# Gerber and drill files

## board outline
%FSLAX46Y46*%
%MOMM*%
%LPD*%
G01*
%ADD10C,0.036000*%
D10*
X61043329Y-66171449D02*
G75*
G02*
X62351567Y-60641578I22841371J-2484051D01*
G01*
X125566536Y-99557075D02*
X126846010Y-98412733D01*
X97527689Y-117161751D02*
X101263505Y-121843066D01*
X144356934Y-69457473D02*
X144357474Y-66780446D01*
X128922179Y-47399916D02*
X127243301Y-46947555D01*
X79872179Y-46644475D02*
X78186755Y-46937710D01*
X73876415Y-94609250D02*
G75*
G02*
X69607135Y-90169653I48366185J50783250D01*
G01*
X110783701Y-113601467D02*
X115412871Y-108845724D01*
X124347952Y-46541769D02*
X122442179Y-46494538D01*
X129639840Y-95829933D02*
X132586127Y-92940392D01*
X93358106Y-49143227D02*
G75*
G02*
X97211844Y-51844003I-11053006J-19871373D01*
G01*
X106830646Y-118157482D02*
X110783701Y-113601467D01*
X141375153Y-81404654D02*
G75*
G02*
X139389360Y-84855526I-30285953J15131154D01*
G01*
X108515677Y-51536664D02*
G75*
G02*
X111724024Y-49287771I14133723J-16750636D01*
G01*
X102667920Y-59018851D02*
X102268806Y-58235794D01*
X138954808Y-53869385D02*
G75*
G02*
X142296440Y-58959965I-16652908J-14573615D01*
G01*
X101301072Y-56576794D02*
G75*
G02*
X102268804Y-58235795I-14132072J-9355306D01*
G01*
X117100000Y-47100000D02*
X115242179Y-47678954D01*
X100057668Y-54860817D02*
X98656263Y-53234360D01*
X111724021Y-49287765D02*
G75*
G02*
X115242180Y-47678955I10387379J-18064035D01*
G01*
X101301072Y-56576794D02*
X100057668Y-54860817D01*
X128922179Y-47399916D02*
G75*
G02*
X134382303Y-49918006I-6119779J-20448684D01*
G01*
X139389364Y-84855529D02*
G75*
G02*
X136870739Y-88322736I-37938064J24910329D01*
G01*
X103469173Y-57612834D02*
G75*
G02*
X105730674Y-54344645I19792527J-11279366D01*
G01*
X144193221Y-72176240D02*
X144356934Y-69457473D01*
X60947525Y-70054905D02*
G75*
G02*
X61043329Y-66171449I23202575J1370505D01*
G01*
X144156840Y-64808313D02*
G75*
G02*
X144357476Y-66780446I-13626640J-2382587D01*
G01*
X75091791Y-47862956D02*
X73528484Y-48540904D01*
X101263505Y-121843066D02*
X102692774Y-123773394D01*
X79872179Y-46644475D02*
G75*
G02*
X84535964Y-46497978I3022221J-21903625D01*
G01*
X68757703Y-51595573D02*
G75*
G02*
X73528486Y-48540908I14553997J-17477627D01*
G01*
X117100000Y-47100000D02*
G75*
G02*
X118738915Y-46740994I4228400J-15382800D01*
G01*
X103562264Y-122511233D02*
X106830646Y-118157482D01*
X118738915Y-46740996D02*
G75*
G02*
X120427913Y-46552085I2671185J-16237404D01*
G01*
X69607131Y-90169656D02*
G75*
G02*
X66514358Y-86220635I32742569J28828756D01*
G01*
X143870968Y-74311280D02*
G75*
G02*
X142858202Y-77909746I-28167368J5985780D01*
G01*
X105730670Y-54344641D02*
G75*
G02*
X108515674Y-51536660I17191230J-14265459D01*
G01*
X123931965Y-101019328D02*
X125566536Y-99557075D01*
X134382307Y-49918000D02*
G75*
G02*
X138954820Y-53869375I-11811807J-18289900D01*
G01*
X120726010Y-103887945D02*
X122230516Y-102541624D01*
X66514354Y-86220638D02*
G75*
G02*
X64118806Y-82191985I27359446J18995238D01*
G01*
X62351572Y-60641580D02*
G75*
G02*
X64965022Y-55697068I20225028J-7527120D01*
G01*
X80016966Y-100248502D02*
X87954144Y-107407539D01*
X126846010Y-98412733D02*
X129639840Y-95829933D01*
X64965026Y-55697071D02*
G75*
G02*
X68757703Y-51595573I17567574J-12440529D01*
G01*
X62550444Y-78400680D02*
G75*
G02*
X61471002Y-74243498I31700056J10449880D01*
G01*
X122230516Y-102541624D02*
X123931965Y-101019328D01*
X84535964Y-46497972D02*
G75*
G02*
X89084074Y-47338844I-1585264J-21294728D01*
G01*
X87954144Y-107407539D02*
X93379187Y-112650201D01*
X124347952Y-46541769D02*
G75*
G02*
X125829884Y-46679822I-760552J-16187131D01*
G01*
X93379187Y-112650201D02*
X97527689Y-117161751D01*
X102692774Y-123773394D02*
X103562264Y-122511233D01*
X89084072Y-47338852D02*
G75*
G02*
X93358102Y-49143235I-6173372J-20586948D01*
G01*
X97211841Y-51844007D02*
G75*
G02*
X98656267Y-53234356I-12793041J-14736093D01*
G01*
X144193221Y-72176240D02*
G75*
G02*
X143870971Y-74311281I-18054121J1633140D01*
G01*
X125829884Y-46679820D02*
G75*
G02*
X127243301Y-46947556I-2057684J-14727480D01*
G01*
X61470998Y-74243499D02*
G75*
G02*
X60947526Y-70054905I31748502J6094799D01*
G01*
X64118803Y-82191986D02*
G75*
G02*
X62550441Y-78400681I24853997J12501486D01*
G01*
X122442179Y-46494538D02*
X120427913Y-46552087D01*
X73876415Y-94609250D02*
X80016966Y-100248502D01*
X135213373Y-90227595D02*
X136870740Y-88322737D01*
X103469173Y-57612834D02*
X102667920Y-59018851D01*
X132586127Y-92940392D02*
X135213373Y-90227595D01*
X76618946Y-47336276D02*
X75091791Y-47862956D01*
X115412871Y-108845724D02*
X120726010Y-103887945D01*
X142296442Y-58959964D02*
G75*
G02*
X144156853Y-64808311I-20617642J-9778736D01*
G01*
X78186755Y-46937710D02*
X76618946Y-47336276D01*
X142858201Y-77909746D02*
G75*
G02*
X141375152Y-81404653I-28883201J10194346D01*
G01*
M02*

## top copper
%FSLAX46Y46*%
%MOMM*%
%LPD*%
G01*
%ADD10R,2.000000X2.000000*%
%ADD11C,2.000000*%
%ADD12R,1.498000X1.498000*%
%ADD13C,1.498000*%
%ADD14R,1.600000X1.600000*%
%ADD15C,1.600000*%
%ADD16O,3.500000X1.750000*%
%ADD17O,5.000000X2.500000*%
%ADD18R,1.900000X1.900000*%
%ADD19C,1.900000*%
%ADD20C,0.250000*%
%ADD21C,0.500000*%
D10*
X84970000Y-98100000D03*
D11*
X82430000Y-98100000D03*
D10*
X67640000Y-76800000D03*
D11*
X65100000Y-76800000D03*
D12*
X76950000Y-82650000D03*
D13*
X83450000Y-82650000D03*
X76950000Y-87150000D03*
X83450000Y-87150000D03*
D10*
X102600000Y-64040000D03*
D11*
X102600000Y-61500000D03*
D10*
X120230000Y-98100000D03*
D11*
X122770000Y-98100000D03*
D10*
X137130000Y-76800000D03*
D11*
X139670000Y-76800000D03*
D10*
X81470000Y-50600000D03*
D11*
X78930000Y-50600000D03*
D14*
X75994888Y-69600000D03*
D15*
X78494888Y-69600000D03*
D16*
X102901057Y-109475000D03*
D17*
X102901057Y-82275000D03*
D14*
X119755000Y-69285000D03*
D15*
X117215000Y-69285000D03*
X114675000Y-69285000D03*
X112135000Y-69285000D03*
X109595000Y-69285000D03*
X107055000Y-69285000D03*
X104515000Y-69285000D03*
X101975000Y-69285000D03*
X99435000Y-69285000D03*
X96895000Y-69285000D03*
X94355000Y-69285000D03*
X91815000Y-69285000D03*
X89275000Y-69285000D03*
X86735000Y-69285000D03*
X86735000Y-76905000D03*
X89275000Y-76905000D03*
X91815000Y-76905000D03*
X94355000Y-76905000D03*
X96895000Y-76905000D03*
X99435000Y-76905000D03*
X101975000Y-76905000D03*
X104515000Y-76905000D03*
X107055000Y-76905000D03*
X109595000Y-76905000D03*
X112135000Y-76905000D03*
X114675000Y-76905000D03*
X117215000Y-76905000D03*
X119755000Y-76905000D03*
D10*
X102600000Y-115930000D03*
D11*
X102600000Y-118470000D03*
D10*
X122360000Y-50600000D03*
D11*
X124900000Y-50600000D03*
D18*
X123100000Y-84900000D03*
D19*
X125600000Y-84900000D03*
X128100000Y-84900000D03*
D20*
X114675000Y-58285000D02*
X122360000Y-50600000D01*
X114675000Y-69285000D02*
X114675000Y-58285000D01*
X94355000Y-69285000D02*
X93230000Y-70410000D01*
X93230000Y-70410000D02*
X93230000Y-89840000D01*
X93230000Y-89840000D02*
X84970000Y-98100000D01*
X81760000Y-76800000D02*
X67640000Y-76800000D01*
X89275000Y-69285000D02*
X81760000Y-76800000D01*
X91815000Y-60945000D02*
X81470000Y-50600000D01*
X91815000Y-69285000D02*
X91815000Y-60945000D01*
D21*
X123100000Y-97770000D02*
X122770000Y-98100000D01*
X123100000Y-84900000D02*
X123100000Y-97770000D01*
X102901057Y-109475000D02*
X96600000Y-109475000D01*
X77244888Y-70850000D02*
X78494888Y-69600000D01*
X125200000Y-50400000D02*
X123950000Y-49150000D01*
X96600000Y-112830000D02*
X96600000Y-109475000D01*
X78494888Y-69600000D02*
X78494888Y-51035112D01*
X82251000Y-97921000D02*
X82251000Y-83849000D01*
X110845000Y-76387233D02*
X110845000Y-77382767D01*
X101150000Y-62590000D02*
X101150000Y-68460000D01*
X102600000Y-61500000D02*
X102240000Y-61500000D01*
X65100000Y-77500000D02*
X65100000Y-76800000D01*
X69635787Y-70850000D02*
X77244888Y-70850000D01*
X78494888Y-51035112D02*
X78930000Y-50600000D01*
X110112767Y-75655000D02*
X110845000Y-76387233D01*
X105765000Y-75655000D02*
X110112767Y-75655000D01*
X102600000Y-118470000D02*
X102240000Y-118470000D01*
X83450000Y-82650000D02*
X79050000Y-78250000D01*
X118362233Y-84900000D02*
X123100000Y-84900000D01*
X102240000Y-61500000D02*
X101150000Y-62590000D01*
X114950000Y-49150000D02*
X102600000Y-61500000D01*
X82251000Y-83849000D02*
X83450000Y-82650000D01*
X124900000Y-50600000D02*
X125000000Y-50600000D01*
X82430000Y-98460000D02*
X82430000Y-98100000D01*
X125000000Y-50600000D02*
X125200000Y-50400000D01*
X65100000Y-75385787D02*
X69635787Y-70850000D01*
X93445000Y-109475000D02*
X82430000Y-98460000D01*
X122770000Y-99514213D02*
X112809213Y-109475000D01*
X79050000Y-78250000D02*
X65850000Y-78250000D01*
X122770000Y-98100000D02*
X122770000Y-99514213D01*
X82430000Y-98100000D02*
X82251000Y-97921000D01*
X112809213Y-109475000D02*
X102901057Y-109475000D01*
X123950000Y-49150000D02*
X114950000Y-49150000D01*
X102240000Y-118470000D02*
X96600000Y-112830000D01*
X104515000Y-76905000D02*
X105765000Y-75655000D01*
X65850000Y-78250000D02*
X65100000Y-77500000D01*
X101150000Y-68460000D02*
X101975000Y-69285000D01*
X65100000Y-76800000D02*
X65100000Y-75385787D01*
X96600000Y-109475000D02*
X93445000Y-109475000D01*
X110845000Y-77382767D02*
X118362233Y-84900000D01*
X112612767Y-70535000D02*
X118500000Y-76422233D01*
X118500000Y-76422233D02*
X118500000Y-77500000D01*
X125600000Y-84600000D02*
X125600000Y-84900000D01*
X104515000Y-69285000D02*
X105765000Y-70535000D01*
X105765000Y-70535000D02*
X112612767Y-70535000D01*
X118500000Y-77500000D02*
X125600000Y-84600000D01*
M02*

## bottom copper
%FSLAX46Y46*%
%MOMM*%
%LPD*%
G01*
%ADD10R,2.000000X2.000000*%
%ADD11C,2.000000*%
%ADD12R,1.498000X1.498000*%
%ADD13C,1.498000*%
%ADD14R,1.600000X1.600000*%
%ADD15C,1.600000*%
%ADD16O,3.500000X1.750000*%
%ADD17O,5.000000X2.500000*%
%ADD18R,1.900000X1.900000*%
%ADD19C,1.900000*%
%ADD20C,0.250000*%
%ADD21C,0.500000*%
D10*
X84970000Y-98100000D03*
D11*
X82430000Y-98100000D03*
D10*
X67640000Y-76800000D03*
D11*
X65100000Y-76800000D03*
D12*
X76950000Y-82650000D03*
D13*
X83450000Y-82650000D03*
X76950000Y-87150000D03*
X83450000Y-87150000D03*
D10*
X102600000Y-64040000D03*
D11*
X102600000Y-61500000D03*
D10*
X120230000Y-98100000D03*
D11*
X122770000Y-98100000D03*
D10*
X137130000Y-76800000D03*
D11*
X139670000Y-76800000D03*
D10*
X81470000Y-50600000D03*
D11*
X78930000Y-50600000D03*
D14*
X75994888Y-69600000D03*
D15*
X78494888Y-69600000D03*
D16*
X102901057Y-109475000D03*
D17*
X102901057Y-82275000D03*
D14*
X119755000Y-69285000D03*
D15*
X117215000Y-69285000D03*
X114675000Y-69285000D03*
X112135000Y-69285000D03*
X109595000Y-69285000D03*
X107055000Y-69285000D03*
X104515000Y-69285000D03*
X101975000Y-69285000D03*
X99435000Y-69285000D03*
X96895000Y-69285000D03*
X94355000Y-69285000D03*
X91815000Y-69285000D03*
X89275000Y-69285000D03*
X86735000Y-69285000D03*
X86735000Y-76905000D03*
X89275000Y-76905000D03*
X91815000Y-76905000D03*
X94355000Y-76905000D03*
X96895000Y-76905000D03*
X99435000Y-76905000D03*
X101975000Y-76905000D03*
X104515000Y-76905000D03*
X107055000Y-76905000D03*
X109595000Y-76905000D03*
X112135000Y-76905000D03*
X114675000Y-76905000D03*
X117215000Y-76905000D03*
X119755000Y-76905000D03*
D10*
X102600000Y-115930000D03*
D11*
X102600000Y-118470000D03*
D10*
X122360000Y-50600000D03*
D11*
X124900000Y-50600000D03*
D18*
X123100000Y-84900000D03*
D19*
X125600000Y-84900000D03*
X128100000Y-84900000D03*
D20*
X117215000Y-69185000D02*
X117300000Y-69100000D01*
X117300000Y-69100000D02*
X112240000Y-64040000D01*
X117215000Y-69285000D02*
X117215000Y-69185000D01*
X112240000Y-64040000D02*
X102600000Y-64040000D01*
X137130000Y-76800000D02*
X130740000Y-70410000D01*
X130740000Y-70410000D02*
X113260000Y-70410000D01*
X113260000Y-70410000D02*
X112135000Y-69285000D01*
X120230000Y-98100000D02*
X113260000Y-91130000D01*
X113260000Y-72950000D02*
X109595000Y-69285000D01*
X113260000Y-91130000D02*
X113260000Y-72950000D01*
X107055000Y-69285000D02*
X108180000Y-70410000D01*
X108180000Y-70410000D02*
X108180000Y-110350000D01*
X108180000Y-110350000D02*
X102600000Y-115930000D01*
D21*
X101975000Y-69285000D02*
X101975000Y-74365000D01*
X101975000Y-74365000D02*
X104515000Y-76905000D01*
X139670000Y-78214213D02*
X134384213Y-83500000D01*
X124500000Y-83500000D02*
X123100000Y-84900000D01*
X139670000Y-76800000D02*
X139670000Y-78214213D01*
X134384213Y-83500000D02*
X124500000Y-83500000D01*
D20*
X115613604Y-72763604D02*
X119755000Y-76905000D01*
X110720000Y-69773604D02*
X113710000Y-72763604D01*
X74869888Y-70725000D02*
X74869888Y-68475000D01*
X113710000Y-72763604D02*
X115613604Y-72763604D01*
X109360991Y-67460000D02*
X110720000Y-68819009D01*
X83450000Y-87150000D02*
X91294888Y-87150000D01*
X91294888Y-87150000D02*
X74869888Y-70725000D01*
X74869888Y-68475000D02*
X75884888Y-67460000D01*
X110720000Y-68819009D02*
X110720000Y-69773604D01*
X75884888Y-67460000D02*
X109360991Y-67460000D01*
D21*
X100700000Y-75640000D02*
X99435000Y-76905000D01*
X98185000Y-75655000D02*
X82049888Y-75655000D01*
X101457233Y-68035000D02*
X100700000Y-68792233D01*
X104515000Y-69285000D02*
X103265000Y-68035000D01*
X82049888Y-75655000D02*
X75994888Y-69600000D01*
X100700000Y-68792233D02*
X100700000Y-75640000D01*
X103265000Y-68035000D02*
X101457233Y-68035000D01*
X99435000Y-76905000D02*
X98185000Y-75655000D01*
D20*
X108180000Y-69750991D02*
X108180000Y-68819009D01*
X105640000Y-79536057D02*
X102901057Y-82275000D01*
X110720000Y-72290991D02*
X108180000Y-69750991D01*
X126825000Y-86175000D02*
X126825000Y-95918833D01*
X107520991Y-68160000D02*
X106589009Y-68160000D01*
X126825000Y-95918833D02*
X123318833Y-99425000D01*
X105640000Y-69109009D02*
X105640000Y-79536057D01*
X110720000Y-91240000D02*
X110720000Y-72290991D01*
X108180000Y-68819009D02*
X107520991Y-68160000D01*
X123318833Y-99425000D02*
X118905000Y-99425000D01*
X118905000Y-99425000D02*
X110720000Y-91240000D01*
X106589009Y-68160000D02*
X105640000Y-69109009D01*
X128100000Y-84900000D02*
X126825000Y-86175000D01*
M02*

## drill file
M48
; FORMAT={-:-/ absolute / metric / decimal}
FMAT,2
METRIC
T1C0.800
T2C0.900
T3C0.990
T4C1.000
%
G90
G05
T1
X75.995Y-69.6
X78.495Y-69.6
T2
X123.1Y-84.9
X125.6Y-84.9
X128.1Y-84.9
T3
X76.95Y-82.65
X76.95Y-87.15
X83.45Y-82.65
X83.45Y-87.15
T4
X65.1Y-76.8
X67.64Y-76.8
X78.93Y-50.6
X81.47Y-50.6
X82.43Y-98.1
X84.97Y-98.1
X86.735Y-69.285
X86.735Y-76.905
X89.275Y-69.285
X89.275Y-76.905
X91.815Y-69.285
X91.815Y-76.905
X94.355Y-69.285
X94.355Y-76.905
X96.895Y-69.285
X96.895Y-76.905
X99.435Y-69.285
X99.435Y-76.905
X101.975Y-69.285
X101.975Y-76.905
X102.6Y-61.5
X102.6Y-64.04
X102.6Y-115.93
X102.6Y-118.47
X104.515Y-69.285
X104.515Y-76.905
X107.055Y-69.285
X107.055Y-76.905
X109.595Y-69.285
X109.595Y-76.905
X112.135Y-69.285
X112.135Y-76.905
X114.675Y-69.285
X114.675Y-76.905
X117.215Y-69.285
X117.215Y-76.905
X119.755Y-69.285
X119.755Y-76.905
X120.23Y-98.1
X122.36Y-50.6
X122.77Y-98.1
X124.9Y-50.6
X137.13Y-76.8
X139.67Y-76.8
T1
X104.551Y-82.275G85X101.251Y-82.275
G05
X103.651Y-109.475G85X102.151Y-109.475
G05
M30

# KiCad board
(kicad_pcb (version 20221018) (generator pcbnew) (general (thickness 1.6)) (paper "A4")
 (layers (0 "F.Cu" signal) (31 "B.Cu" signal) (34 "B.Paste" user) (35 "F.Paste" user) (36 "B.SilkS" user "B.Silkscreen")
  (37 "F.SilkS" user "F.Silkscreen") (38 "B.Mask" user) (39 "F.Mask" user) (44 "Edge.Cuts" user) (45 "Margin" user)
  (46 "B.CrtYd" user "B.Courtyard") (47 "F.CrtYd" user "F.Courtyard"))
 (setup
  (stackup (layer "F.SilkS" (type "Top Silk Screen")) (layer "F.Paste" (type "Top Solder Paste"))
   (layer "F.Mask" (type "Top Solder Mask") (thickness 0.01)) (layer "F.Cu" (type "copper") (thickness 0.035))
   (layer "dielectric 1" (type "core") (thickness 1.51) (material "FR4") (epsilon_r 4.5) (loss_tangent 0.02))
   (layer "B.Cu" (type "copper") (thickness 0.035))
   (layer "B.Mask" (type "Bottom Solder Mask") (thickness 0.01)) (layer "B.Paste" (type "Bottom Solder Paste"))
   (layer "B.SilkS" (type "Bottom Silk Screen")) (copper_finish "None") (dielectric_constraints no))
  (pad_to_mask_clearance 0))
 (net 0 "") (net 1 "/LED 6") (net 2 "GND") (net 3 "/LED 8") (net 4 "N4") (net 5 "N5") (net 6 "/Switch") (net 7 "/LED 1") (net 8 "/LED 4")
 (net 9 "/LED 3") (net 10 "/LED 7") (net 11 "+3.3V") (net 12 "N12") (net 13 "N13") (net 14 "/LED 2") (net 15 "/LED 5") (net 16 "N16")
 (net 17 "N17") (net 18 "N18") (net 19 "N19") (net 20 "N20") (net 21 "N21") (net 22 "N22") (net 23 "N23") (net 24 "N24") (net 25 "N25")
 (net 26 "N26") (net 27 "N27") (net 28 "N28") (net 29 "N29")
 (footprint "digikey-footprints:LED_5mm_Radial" (layer "F.Cu") (at 82.43 98.1 180)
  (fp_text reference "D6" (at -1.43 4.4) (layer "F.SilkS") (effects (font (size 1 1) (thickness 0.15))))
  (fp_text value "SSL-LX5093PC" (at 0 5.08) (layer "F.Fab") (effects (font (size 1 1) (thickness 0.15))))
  (pad "1" thru_hole rect (at -2.54 0 180) (size 2 2) (drill 1) (layers "*.Cu" "*.Mask") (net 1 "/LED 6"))
  (pad "2" thru_hole circle (at 0 0 180) (size 2 2) (drill 1) (layers "*.Cu" "*.Mask") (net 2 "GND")))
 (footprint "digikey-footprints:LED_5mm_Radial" (layer "F.Cu") (at 65.1 76.8 180)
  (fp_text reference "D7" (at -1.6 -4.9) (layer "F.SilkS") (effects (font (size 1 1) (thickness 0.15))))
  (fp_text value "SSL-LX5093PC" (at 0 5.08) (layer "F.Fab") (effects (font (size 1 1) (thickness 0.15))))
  (pad "1" thru_hole rect (at -2.54 0 180) (size 2 2) (drill 1) (layers "*.Cu" "*.Mask") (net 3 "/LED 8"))
  (pad "2" thru_hole circle (at 0 0 180) (size 2 2) (drill 1) (layers "*.Cu" "*.Mask") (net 2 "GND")))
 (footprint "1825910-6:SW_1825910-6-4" (layer "F.Cu") (at 80.2 84.9)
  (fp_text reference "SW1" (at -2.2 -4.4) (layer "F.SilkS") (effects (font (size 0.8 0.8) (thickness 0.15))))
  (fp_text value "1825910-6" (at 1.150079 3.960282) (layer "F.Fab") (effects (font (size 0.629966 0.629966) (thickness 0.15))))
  (pad "1" thru_hole rect (at -3.25 -2.25) (size 1.498 1.498) (drill 0.99) (layers "*.Cu" "*.Mask") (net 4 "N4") (solder_mask_margin 0.102))
  (pad "2" thru_hole circle (at 3.25 -2.25) (size 1.498 1.498) (drill 0.99) (layers "*.Cu" "*.Mask") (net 2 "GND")
   (solder_mask_margin 0.102))
  (pad "3" thru_hole circle (at -3.25 2.25) (size 1.498 1.498) (drill 0.99) (layers "*.Cu" "*.Mask") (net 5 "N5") (solder_mask_margin 0.102))
  (pad "4" thru_hole circle (at 3.25 2.25) (size 1.498 1.498) (drill 0.99) (layers "*.Cu" "*.Mask") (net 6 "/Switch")
   (solder_mask_margin 0.102)))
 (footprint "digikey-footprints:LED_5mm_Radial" (layer "F.Cu") (at 102.6 61.5 90)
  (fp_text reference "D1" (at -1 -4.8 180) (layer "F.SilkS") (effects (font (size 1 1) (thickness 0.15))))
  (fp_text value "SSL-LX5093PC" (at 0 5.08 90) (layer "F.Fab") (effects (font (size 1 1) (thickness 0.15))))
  (pad "1" thru_hole rect (at -2.54 0 90) (size 2 2) (drill 1) (layers "*.Cu" "*.Mask") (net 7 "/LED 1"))
  (pad "2" thru_hole circle (at 0 0 90) (size 2 2) (drill 1) (layers "*.Cu" "*.Mask") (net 2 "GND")))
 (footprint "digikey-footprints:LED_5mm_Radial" (layer "F.Cu") (at 122.77 98.1)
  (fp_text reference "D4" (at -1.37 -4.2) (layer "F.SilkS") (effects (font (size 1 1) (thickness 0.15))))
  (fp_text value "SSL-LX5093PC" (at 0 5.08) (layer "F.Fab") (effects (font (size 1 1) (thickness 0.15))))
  (pad "1" thru_hole rect (at -2.54 0) (size 2 2) (drill 1) (layers "*.Cu" "*.Mask") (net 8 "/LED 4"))
  (pad "2" thru_hole circle (at 0 0) (size 2 2) (drill 1) (layers "*.Cu" "*.Mask") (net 2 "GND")))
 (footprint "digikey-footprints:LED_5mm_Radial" (layer "F.Cu") (at 139.67 76.8)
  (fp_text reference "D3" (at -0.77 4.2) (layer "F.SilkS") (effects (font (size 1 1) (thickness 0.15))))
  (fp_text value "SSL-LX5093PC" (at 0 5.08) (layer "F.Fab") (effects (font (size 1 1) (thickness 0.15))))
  (pad "1" thru_hole rect (at -2.54 0) (size 2 2) (drill 1) (layers "*.Cu" "*.Mask") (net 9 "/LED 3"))
  (pad "2" thru_hole circle (at 0 0) (size 2 2) (drill 1) (layers "*.Cu" "*.Mask") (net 2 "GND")))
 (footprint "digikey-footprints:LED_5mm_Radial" (layer "F.Cu") (at 78.93 50.6 180)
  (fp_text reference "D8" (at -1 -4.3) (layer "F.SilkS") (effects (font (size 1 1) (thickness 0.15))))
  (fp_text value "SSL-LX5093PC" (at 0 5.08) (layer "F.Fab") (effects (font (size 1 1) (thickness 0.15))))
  (pad "1" thru_hole rect (at -2.54 0 180) (size 2 2) (drill 1) (layers "*.Cu" "*.Mask") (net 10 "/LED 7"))
  (pad "2" thru_hole circle (at 0 0 180) (size 2 2) (drill 1) (layers "*.Cu" "*.Mask") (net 2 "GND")))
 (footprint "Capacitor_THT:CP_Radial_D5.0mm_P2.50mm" (layer "F.Cu") (at 75.994888 69.6)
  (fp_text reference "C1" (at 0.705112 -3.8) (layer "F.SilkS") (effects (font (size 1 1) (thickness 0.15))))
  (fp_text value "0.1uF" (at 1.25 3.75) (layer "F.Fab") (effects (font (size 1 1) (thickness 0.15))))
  (pad "1" thru_hole rect (at 0 0) (size 1.6 1.6) (drill 0.8) (layers "*.Cu" "*.Mask") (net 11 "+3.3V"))
  (pad "2" thru_hole circle (at 2.5 0) (size 1.6 1.6) (drill 0.8) (layers "*.Cu" "*.Mask") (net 2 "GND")))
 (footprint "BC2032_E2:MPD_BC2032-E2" (layer "F.Cu") (at 102.901057 95.875 -90)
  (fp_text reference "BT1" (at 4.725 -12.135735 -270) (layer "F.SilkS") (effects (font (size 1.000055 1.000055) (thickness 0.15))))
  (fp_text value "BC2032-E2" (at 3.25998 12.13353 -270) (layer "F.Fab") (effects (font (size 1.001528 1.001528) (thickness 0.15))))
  (pad "N" thru_hole oval (at 13.6 0 270) (size 1.75 3.5) (drill oval 0.8 2.3) (layers "*.Cu" "*.Mask") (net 2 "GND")
   (solder_mask_margin 0.102))
  (pad "P" thru_hole oval (at -13.6 0 270) (size 2.5 5) (drill oval 0.8 4.1) (layers "*.Cu" "*.Mask") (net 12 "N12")
   (solder_mask_margin 0.102)))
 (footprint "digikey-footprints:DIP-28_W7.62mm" (layer "F.Cu") (at 119.755 69.285 -90)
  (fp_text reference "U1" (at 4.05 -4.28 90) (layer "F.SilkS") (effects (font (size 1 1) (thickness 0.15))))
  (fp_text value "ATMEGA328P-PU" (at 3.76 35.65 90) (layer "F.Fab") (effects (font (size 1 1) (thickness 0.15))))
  (pad "1" thru_hole rect (at 0 0 270) (size 1.6 1.6) (drill 1) (layers "*.Cu" "*.Mask") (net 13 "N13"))
  (pad "2" thru_hole circle (at 0 2.54 270) (size 1.6 1.6) (drill 1) (layers "*.Cu" "*.Mask") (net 7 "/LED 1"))
  (pad "3" thru_hole circle (at 0 5.08 270) (size 1.6 1.6) (drill 1) (layers "*.Cu" "*.Mask") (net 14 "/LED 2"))
  (pad "4" thru_hole circle (at 0 7.62 270) (size 1.6 1.6) (drill 1) (layers "*.Cu" "*.Mask") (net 9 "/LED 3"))
  (pad "5" thru_hole circle (at 0 10.16 270) (size 1.6 1.6) (drill 1) (layers "*.Cu" "*.Mask") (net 8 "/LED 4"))
  (pad "6" thru_hole circle (at 0 12.7 270) (size 1.6 1.6) (drill 1) (layers "*.Cu" "*.Mask") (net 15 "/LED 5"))
  (pad "7" thru_hole circle (at 0 15.24 270) (size 1.6 1.6) (drill 1) (layers "*.Cu" "*.Mask") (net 11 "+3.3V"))
  (pad "8" thru_hole circle (at 0 17.78 270) (size 1.6 1.6) (drill 1) (layers "*.Cu" "*.Mask") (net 2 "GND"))
  (pad "9" thru_hole circle (at 0 20.32 270) (size 1.6 1.6) (drill 1) (layers "*.Cu" "*.Mask") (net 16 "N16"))
  (pad "10" thru_hole circle (at 0 22.86 270) (size 1.6 1.6) (drill 1) (layers "*.Cu" "*.Mask") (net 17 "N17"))
  (pad "11" thru_hole circle (at 0 25.4 270) (size 1.6 1.6) (drill 1) (layers "*.Cu" "*.Mask") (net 1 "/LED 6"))
  (pad "12" thru_hole circle (at 0 27.94 270) (size 1.6 1.6) (drill 1) (layers "*.Cu" "*.Mask") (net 10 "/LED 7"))
  (pad "13" thru_hole circle (at 0 30.48 270) (size 1.6 1.6) (drill 1) (layers "*.Cu" "*.Mask") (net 3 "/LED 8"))
  (pad "14" thru_hole circle (at 0 33.02 270) (size 1.6 1.6) (drill 1) (layers "*.Cu" "*.Mask") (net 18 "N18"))
  (pad "15" thru_hole circle (at 7.62 33.02 270) (size 1.6 1.6) (drill 1) (layers "*.Cu" "*.Mask") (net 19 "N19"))
  (pad "16" thru_hole circle (at 7.62 30.48 270) (size 1.6 1.6) (drill 1) (layers "*.Cu" "*.Mask") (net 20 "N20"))
  (pad "17" thru_hole circle (at 7.62 27.94 270) (size 1.6 1.6) (drill 1) (layers "*.Cu" "*.Mask") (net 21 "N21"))
  (pad "18" thru_hole circle (at 7.62 25.4 270) (size 1.6 1.6) (drill 1) (layers "*.Cu" "*.Mask") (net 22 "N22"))
  (pad "19" thru_hole circle (at 7.62 22.86 270) (size 1.6 1.6) (drill 1) (layers "*.Cu" "*.Mask") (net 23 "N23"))
  (pad "20" thru_hole circle (at 7.62 20.32 270) (size 1.6 1.6) (drill 1) (layers "*.Cu" "*.Mask") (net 11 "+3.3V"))
  (pad "21" thru_hole circle (at 7.62 17.78 270) (size 1.6 1.6) (drill 1) (layers "*.Cu" "*.Mask") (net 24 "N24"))
  (pad "22" thru_hole circle (at 7.62 15.24 270) (size 1.6 1.6) (drill 1) (layers "*.Cu" "*.Mask") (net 2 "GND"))
  (pad "23" thru_hole circle (at 7.62 12.7 270) (size 1.6 1.6) (drill 1) (layers "*.Cu" "*.Mask") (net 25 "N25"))
  (pad "24" thru_hole circle (at 7.62 10.16 270) (size 1.6 1.6) (drill 1) (layers "*.Cu" "*.Mask") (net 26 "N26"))
  (pad "25" thru_hole circle (at 7.62 7.62 270) (size 1.6 1.6) (drill 1) (layers "*.Cu" "*.Mask") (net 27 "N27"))
  (pad "26" thru_hole circle (at 7.62 5.08 270) (size 1.6 1.6) (drill 1) (layers "*.Cu" "*.Mask") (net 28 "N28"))
  (pad "27" thru_hole circle (at 7.62 2.54 270) (size 1.6 1.6) (drill 1) (layers "*.Cu" "*.Mask") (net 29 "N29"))
  (pad "28" thru_hole circle (at 7.62 0 270) (size 1.6 1.6) (drill 1) (layers "*.Cu" "*.Mask") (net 6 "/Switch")))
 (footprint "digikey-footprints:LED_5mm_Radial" (layer "F.Cu") (at 102.6 118.47 -90)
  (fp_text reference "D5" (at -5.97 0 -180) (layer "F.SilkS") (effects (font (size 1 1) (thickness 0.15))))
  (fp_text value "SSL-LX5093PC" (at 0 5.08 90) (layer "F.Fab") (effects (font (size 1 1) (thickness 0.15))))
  (pad "1" thru_hole rect (at -2.54 0 270) (size 2 2) (drill 1) (layers "*.Cu" "*.Mask") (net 15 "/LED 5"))
  (pad "2" thru_hole circle (at 0 0 270) (size 2 2) (drill 1) (layers "*.Cu" "*.Mask") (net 2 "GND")))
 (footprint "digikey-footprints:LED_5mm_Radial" (layer "F.Cu") (at 124.9 50.6)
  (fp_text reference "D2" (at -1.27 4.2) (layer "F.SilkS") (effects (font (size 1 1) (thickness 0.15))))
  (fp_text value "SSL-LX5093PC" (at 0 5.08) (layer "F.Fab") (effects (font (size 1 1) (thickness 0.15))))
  (pad "1" thru_hole rect (at -2.54 0) (size 2 2) (drill 1) (layers "*.Cu" "*.Mask") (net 14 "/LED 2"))
  (pad "2" thru_hole circle (at 0 0) (size 2 2) (drill 1) (layers "*.Cu" "*.Mask") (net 2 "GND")))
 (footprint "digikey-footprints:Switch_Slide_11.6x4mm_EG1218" (layer "F.Cu") (at 123.1 84.9)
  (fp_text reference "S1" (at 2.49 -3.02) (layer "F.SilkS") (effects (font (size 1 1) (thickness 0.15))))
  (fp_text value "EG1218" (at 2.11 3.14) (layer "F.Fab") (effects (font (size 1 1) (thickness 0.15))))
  (pad "1" thru_hole rect (at 0 0) (size 1.9 1.9) (drill 0.9) (layers "*.Cu" "*.Mask") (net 2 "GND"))
  (pad "2" thru_hole circle (at 2.5 0) (size 1.9 1.9) (drill 0.9) (layers "*.Cu" "*.Mask") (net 11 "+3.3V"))
  (pad "3" thru_hole circle (at 5 0) (size 1.9 1.9) (drill 0.9) (layers "*.Cu" "*.Mask") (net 12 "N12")))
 (gr_arc (start 61.043329 66.171449) (mid 61.525834 63.365914) (end 62.351572 60.64158) (stroke (width 0.036) (type solid))
  (layer "Edge.Cuts"))
 (gr_line (start 125.566536 99.557075) (end 126.84601 98.412733) (stroke (width 0.036) (type solid)) (layer "Edge.Cuts"))
 (gr_line (start 97.527689 117.161751) (end 101.263505 121.843066) (stroke (width 0.036) (type solid)) (layer "Edge.Cuts"))
 (gr_line (start 144.356934 69.457473) (end 144.357474 66.780446) (stroke (width 0.036) (type solid)) (layer "Edge.Cuts"))
 (gr_line (start 128.922179 47.399916) (end 127.243301 46.947555) (stroke (width 0.036) (type solid)) (layer "Edge.Cuts"))
 (gr_line (start 79.872179 46.644475) (end 78.186755 46.93771) (stroke (width 0.036) (type solid)) (layer "Edge.Cuts"))
 (gr_arc (start 73.876415 94.60925) (mid 71.69301 92.436345) (end 69.607131 90.169656) (stroke (width 0.036) (type solid))
  (layer "Edge.Cuts"))
 (gr_line (start 110.783701 113.601467) (end 115.412871 108.845724) (stroke (width 0.036) (type solid)) (layer "Edge.Cuts"))
 (gr_line (start 124.347952 46.541769) (end 122.442179 46.494538) (stroke (width 0.036) (type solid)) (layer "Edge.Cuts"))
 (gr_line (start 129.63984 95.829933) (end 132.586127 92.940392) (stroke (width 0.036) (type solid)) (layer "Edge.Cuts"))
 (gr_arc (start 93.358106 49.143227) (mid 95.35503 50.393654) (end 97.211841 51.844007) (stroke (width 0.036) (type solid))
  (layer "Edge.Cuts"))
 (gr_line (start 106.830646 118.157482) (end 110.783701 113.601467) (stroke (width 0.036) (type solid)) (layer "Edge.Cuts"))
 (gr_arc (start 141.375153 81.404654) (mid 140.433031 83.159308) (end 139.389364 84.855529) (stroke (width 0.036) (type solid))
  (layer "Edge.Cuts"))
 (gr_arc (start 108.515677 51.536664) (mid 110.069494 50.340377) (end 111.724021 49.287765) (stroke (width 0.036) (type solid))
  (layer "Edge.Cuts"))
 (gr_line (start 102.66792 59.018851) (end 102.268806 58.235794) (stroke (width 0.036) (type solid)) (layer "Edge.Cuts"))
 (gr_arc (start 138.954808 53.869385) (mid 140.80156 56.299185) (end 142.296442 58.959964) (stroke (width 0.036) (type solid))
  (layer "Edge.Cuts"))
 (gr_arc (start 101.301072 56.576794) (mid 101.808458 57.392574) (end 102.268806 58.235794) (stroke (width 0.036) (type solid))
  (layer "Edge.Cuts"))
 (gr_line (start 117.1 47.1) (end 115.242179 47.678954) (stroke (width 0.036) (type solid)) (layer "Edge.Cuts"))
 (gr_line (start 100.057668 54.860817) (end 98.656263 53.23436) (stroke (width 0.036) (type solid)) (layer "Edge.Cuts"))
 (gr_arc (start 111.724021 49.287765) (mid 113.445684 48.401539) (end 115.242179 47.678954) (stroke (width 0.036) (type solid))
  (layer "Edge.Cuts"))
 (gr_line (start 101.301072 56.576794) (end 100.057668 54.860817) (stroke (width 0.036) (type solid)) (layer "Edge.Cuts"))
 (gr_arc (start 128.922179 47.399916) (mid 131.741355 48.465731) (end 134.382307 49.918) (stroke (width 0.036) (type solid))
  (layer "Edge.Cuts"))
 (gr_arc (start 139.389364 84.855529) (mid 138.170998 86.618877) (end 136.87074 88.322737) (stroke (width 0.036) (type solid))
  (layer "Edge.Cuts"))
 (gr_arc (start 103.469173 57.612834) (mid 104.528514 55.929326) (end 105.73067 54.344641) (stroke (width 0.036) (type solid))
  (layer "Edge.Cuts"))
 (gr_line (start 144.193221 72.17624) (end 144.356934 69.457473) (stroke (width 0.036) (type solid)) (layer "Edge.Cuts"))
 (gr_arc (start 60.947525 70.054905) (mid 60.914154 68.111172) (end 61.043329 66.171449) (stroke (width 0.036) (type solid))
  (layer "Edge.Cuts"))
 (gr_arc (start 144.15684 64.808313) (mid 144.292528 65.790781) (end 144.357474 66.780446) (stroke (width 0.036) (type solid))
  (layer "Edge.Cuts"))
 (gr_line (start 75.091791 47.862956) (end 73.528484 48.540904) (stroke (width 0.036) (type solid)) (layer "Edge.Cuts"))
 (gr_line (start 101.263505 121.843066) (end 102.692774 123.773394) (stroke (width 0.036) (type solid)) (layer "Edge.Cuts"))
 (gr_arc (start 79.872179 46.644475) (mid 82.200196 46.447855) (end 84.535964 46.497972) (stroke (width 0.036) (type solid))
  (layer "Edge.Cuts"))
 (gr_arc (start 68.757703 51.595573) (mid 71.047617 49.919123) (end 73.528484 48.540904) (stroke (width 0.036) (type solid))
  (layer "Edge.Cuts"))
 (gr_arc (start 117.1 47.1) (mid 117.914735 46.898938) (end 118.738915 46.740996) (stroke (width 0.036) (type solid)) (layer "Edge.Cuts"))
 (gr_line (start 103.562264 122.511233) (end 106.830646 118.157482) (stroke (width 0.036) (type solid)) (layer "Edge.Cuts"))
 (gr_arc (start 118.738915 46.740996) (mid 119.580974 46.624722) (end 120.427913 46.552087) (stroke (width 0.036) (type solid))
  (layer "Edge.Cuts"))
 (gr_arc (start 69.607131 90.169656) (mid 68.003939 88.239634) (end 66.514354 86.220638) (stroke (width 0.036) (type solid))
  (layer "Edge.Cuts"))
 (gr_arc (start 143.870968 74.31128) (mid 143.423039 76.126965) (end 142.858201 77.909746) (stroke (width 0.036) (type solid))
  (layer "Edge.Cuts"))
 (gr_arc (start 105.73067 54.344641) (mid 107.060912 52.8789) (end 108.515677 51.536664) (stroke (width 0.036) (type solid))
  (layer "Edge.Cuts"))
 (gr_line (start 123.931965 101.019328) (end 125.566536 99.557075) (stroke (width 0.036) (type solid)) (layer "Edge.Cuts"))
 (gr_arc (start 134.382307 49.918) (mid 136.80632 51.734275) (end 138.954808 53.869385) (stroke (width 0.036) (type solid))
  (layer "Edge.Cuts"))
 (gr_line (start 120.72601 103.887945) (end 122.230516 102.541624) (stroke (width 0.036) (type solid)) (layer "Edge.Cuts"))
 (gr_arc (start 66.514354 86.220638) (mid 65.245625 84.248503) (end 64.118803 82.191986) (stroke (width 0.036) (type solid))
  (layer "Edge.Cuts"))
 (gr_arc (start 62.351572 60.64158) (mid 63.497445 58.084305) (end 64.965026 55.697071) (stroke (width 0.036) (type solid))
  (layer "Edge.Cuts"))
 (gr_line (start 80.016966 100.248502) (end 87.954144 107.407539) (stroke (width 0.036) (type solid)) (layer "Edge.Cuts"))
 (gr_line (start 126.84601 98.412733) (end 129.63984 95.829933) (stroke (width 0.036) (type solid)) (layer "Edge.Cuts"))
 (gr_arc (start 64.965026 55.697071) (mid 66.727753 53.52277) (end 68.757703 51.595573) (stroke (width 0.036) (type solid))
  (layer "Edge.Cuts"))
 (gr_arc (start 62.550444 78.40068) (mid 61.943784 76.33947) (end 61.470998 74.243499) (stroke (width 0.036) (type solid))
  (layer "Edge.Cuts"))
 (gr_line (start 122.230516 102.541624) (end 123.931965 101.019328) (stroke (width 0.036) (type solid)) (layer "Edge.Cuts"))
 (gr_arc (start 84.535964 46.497972) (mid 86.832852 46.794909) (end 89.084072 47.338852) (stroke (width 0.036) (type solid))
  (layer "Edge.Cuts"))
 (gr_line (start 87.954144 107.407539) (end 93.379187 112.650201) (stroke (width 0.036) (type solid)) (layer "Edge.Cuts"))
 (gr_arc (start 124.347952 46.541769) (mid 125.090504 46.593772) (end 125.829884 46.67982) (stroke (width 0.036) (type solid))
  (layer "Edge.Cuts"))
 (gr_line (start 93.379187 112.650201) (end 97.527689 117.161751) (stroke (width 0.036) (type solid)) (layer "Edge.Cuts"))
 (gr_line (start 102.692774 123.773394) (end 103.562264 122.511233) (stroke (width 0.036) (type solid)) (layer "Edge.Cuts"))
 (gr_arc (start 89.084072 47.338852) (mid 91.269917 48.12538) (end 93.358106 49.143227) (stroke (width 0.036) (type solid))
  (layer "Edge.Cuts"))
 (gr_arc (start 97.211841 51.844007) (mid 97.951919 52.520622) (end 98.656263 53.23436) (stroke (width 0.036) (type solid))
  (layer "Edge.Cuts"))
 (gr_arc (start 144.193221 72.17624) (mid 144.063911 73.248562) (end 143.870968 74.31128) (stroke (width 0.036) (type solid))
  (layer "Edge.Cuts"))
 (gr_arc (start 125.829884 46.67982) (mid 126.539832 46.796586) (end 127.243301 46.947555) (stroke (width 0.036) (type solid))
  (layer "Edge.Cuts"))
 (gr_arc (start 61.470998 74.243499) (mid 61.140824 72.157755) (end 60.947525 70.054905) (stroke (width 0.036) (type solid))
  (layer "Edge.Cuts"))
 (gr_arc (start 64.118803 82.191986) (mid 63.264638 80.325284) (end 62.550444 78.40068) (stroke (width 0.036) (type solid))
  (layer "Edge.Cuts"))
 (gr_line (start 122.442179 46.494538) (end 120.427913 46.552087) (stroke (width 0.036) (type solid)) (layer "Edge.Cuts"))
 (gr_line (start 73.876415 94.60925) (end 80.016966 100.248502) (stroke (width 0.036) (type solid)) (layer "Edge.Cuts"))
 (gr_line (start 135.213373 90.227595) (end 136.87074 88.322737) (stroke (width 0.036) (type solid)) (layer "Edge.Cuts"))
 (gr_line (start 103.469173 57.612834) (end 102.66792 59.018851) (stroke (width 0.036) (type solid)) (layer "Edge.Cuts"))
 (gr_line (start 132.586127 92.940392) (end 135.213373 90.227595) (stroke (width 0.036) (type solid)) (layer "Edge.Cuts"))
 (gr_line (start 76.618946 47.336276) (end 75.091791 47.862956) (stroke (width 0.036) (type solid)) (layer "Edge.Cuts"))
 (gr_line (start 115.412871 108.845724) (end 120.72601 103.887945) (stroke (width 0.036) (type solid)) (layer "Edge.Cuts"))
 (gr_arc (start 142.296442 58.959964) (mid 143.42415 61.82131) (end 144.15684 64.808313) (stroke (width 0.036) (type solid))
  (layer "Edge.Cuts"))
 (gr_line (start 78.186755 46.93771) (end 76.618946 47.336276) (stroke (width 0.036) (type solid)) (layer "Edge.Cuts"))
 (gr_arc (start 142.858201 77.909746) (mid 142.170879 79.6802) (end 141.375153 81.404654) (stroke (width 0.036) (type solid))
  (layer "Edge.Cuts"))
 (segment (start 117.215 69.185) (end 117.3 69.1) (width 0.25) (layer "B.Cu") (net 7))
 (segment (start 117.3 69.1) (end 112.24 64.04) (width 0.25) (layer "B.Cu") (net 7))
 (segment (start 117.215 69.285) (end 117.215 69.185) (width 0.25) (layer "B.Cu") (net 7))
 (segment (start 112.24 64.04) (end 102.6 64.04) (width 0.25) (layer "B.Cu") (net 7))
 (segment (start 114.675 58.285) (end 122.36 50.6) (width 0.25) (layer "F.Cu") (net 14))
 (segment (start 114.675 69.285) (end 114.675 58.285) (width 0.25) (layer "F.Cu") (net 14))
 (segment (start 137.13 76.8) (end 130.74 70.41) (width 0.25) (layer "B.Cu") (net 9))
 (segment (start 130.74 70.41) (end 113.26 70.41) (width 0.25) (layer "B.Cu") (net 9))
 (segment (start 113.26 70.41) (end 112.135 69.285) (width 0.25) (layer "B.Cu") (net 9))
 (segment (start 120.23 98.1) (end 113.26 91.13) (width 0.25) (layer "B.Cu") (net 8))
 (segment (start 113.26 72.95) (end 109.595 69.285) (width 0.25) (layer "B.Cu") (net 8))
 (segment (start 113.26 91.13) (end 113.26 72.95) (width 0.25) (layer "B.Cu") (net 8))
 (segment (start 107.055 69.285) (end 108.18 70.41) (width 0.25) (layer "B.Cu") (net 15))
 (segment (start 108.18 70.41) (end 108.18 110.35) (width 0.25) (layer "B.Cu") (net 15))
 (segment (start 108.18 110.35) (end 102.6 115.93) (width 0.25) (layer "B.Cu") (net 15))
 (segment (start 94.355 69.285) (end 93.23 70.41) (width 0.25) (layer "F.Cu") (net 1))
 (segment (start 93.23 70.41) (end 93.23 89.84) (width 0.25) (layer "F.Cu") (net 1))
 (segment (start 93.23 89.84) (end 84.97 98.1) (width 0.25) (layer "F.Cu") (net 1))
 (segment (start 81.76 76.8) (end 67.64 76.8) (width 0.25) (layer "F.Cu") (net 3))
 (segment (start 89.275 69.285) (end 81.76 76.8) (width 0.25) (layer "F.Cu") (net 3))
 (segment (start 91.815 60.945) (end 81.47 50.6) (width 0.25) (layer "F.Cu") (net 10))
 (segment (start 91.815 69.285) (end 91.815 60.945) (width 0.25) (layer "F.Cu") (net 10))
 (segment (start 123.1 97.77) (end 122.77 98.1) (width 0.5) (layer "F.Cu") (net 2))
 (segment (start 123.1 84.9) (end 123.1 97.77) (width 0.5) (layer "F.Cu") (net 2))
 (segment (start 102.901057 109.475) (end 96.6 109.475) (width 0.5) (layer "F.Cu") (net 2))
 (segment (start 77.244888 70.85) (end 78.494888 69.6) (width 0.5) (layer "F.Cu") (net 2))
 (segment (start 125.2 50.4) (end 123.95 49.15) (width 0.5) (layer "F.Cu") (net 2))
 (segment (start 96.6 112.83) (end 96.6 109.475) (width 0.5) (layer "F.Cu") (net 2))
 (segment (start 78.494888 69.6) (end 78.494888 51.035112) (width 0.5) (layer "F.Cu") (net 2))
 (segment (start 82.251 97.921) (end 82.251 83.849) (width 0.5) (layer "F.Cu") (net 2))
 (segment (start 110.845 76.387233) (end 110.845 77.382767) (width 0.5) (layer "F.Cu") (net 2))
 (segment (start 101.15 62.59) (end 101.15 68.46) (width 0.5) (layer "F.Cu") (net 2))
 (segment (start 102.6 61.5) (end 102.24 61.5) (width 0.5) (layer "F.Cu") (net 2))
 (segment (start 65.1 77.5) (end 65.1 76.8) (width 0.5) (layer "F.Cu") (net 2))
 (segment (start 69.635787 70.85) (end 77.244888 70.85) (width 0.5) (layer "F.Cu") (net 2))
 (segment (start 78.494888 51.035112) (end 78.93 50.6) (width 0.5) (layer "F.Cu") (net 2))
 (segment (start 110.112767 75.655) (end 110.845 76.387233) (width 0.5) (layer "F.Cu") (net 2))
 (segment (start 105.765 75.655) (end 110.112767 75.655) (width 0.5) (layer "F.Cu") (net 2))
 (segment (start 102.6 118.47) (end 102.24 118.47) (width 0.5) (layer "F.Cu") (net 2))
 (segment (start 83.45 82.65) (end 79.05 78.25) (width 0.5) (layer "F.Cu") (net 2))
 (segment (start 118.362233 84.9) (end 123.1 84.9) (width 0.5) (layer "F.Cu") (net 2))
 (segment (start 102.24 61.5) (end 101.15 62.59) (width 0.5) (layer "F.Cu") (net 2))
 (segment (start 114.95 49.15) (end 102.6 61.5) (width 0.5) (layer "F.Cu") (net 2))
 (segment (start 82.251 83.849) (end 83.45 82.65) (width 0.5) (layer "F.Cu") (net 2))
 (segment (start 124.9 50.6) (end 125 50.6) (width 0.5) (layer "F.Cu") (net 2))
 (segment (start 82.43 98.46) (end 82.43 98.1) (width 0.5) (layer "F.Cu") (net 2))
 (segment (start 125 50.6) (end 125.2 50.4) (width 0.5) (layer "F.Cu") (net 2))
 (segment (start 65.1 75.385787) (end 69.635787 70.85) (width 0.5) (layer "F.Cu") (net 2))
 (segment (start 93.445 109.475) (end 82.43 98.46) (width 0.5) (layer "F.Cu") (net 2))
 (segment (start 122.77 99.514213) (end 112.809213 109.475) (width 0.5) (layer "F.Cu") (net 2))
 (segment (start 79.05 78.25) (end 65.85 78.25) (width 0.5) (layer "F.Cu") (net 2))
 (segment (start 122.77 98.1) (end 122.77 99.514213) (width 0.5) (layer "F.Cu") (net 2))
 (segment (start 82.43 98.1) (end 82.251 97.921) (width 0.5) (layer "F.Cu") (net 2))
 (segment (start 112.809213 109.475) (end 102.901057 109.475) (width 0.5) (layer "F.Cu") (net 2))
 (segment (start 123.95 49.15) (end 114.95 49.15) (width 0.5) (layer "F.Cu") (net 2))
 (segment (start 102.24 118.47) (end 96.6 112.83) (width 0.5) (layer "F.Cu") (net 2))
 (segment (start 104.515 76.905) (end 105.765 75.655) (width 0.5) (layer "F.Cu") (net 2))
 (segment (start 65.85 78.25) (end 65.1 77.5) (width 0.5) (layer "F.Cu") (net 2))
 (segment (start 101.15 68.46) (end 101.975 69.285) (width 0.5) (layer "F.Cu") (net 2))
 (segment (start 65.1 76.8) (end 65.1 75.385787) (width 0.5) (layer "F.Cu") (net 2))
 (segment (start 96.6 109.475) (end 93.445 109.475) (width 0.5) (layer "F.Cu") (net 2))
 (segment (start 110.845 77.382767) (end 118.362233 84.9) (width 0.5) (layer "F.Cu") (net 2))
 (segment (start 101.975 69.285) (end 101.975 74.365) (width 0.5) (layer "B.Cu") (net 2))
 (segment (start 101.975 74.365) (end 104.515 76.905) (width 0.5) (layer "B.Cu") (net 2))
 (segment (start 139.67 78.214213) (end 134.384213 83.5) (width 0.5) (layer "B.Cu") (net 2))
 (segment (start 124.5 83.5) (end 123.1 84.9) (width 0.5) (layer "B.Cu") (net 2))
 (segment (start 139.67 76.8) (end 139.67 78.214213) (width 0.5) (layer "B.Cu") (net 2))
 (segment (start 134.384213 83.5) (end 124.5 83.5) (width 0.5) (layer "B.Cu") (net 2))
 (segment (start 115.613604 72.763604) (end 119.755 76.905) (width 0.25) (layer "B.Cu") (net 6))
 (segment (start 110.72 69.773604) (end 113.71 72.763604) (width 0.25) (layer "B.Cu") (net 6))
 (segment (start 74.869888 70.725) (end 74.869888 68.475) (width 0.25) (layer "B.Cu") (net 6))
 (segment (start 113.71 72.763604) (end 115.613604 72.763604) (width 0.25) (layer "B.Cu") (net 6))
 (segment (start 109.360991 67.46) (end 110.72 68.819009) (width 0.25) (layer "B.Cu") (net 6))
 (segment (start 83.45 87.15) (end 91.294888 87.15) (width 0.25) (layer "B.Cu") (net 6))
 (segment (start 91.294888 87.15) (end 74.869888 70.725) (width 0.25) (layer "B.Cu") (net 6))
 (segment (start 74.869888 68.475) (end 75.884888 67.46) (width 0.25) (layer "B.Cu") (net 6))
 (segment (start 110.72 68.819009) (end 110.72 69.773604) (width 0.25) (layer "B.Cu") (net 6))
 (segment (start 75.884888 67.46) (end 109.360991 67.46) (width 0.25) (layer "B.Cu") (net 6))
 (segment (start 112.612767 70.535) (end 118.5 76.422233) (width 0.5) (layer "F.Cu") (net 11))
 (segment (start 118.5 76.422233) (end 118.5 77.5) (width 0.5) (layer "F.Cu") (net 11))
 (segment (start 125.6 84.6) (end 125.6 84.9) (width 0.5) (layer "F.Cu") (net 11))
 (segment (start 104.515 69.285) (end 105.765 70.535) (width 0.5) (layer "F.Cu") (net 11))
 (segment (start 105.765 70.535) (end 112.612767 70.535) (width 0.5) (layer "F.Cu") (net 11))
 (segment (start 118.5 77.5) (end 125.6 84.6) (width 0.5) (layer "F.Cu") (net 11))
 (segment (start 100.7 75.64) (end 99.435 76.905) (width 0.5) (layer "B.Cu") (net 11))
 (segment (start 98.185 75.655) (end 82.049888 75.655) (width 0.5) (layer "B.Cu") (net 11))
 (segment (start 101.457233 68.035) (end 100.7 68.792233) (width 0.5) (layer "B.Cu") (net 11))
 (segment (start 104.515 69.285) (end 103.265 68.035) (width 0.5) (layer "B.Cu") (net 11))
 (segment (start 82.049888 75.655) (end 75.994888 69.6) (width 0.5) (layer "B.Cu") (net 11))
 (segment (start 100.7 68.792233) (end 100.7 75.64) (width 0.5) (layer "B.Cu") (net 11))
 (segment (start 103.265 68.035) (end 101.457233 68.035) (width 0.5) (layer "B.Cu") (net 11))
 (segment (start 99.435 76.905) (end 98.185 75.655) (width 0.5) (layer "B.Cu") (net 11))
 (segment (start 108.18 69.750991) (end 108.18 68.819009) (width 0.25) (layer "B.Cu") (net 12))
 (segment (start 105.64 79.536057) (end 102.901057 82.275) (width 0.25) (layer "B.Cu") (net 12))
 (segment (start 110.72 72.290991) (end 108.18 69.750991) (width 0.25) (layer "B.Cu") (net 12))
 (segment (start 126.825 86.175) (end 126.825 95.918833) (width 0.25) (layer "B.Cu") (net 12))
 (segment (start 107.520991 68.16) (end 106.589009 68.16) (width 0.25) (layer "B.Cu") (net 12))
 (segment (start 126.825 95.918833) (end 123.318833 99.425) (width 0.25) (layer "B.Cu") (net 12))
 (segment (start 105.64 69.109009) (end 105.64 79.536057) (width 0.25) (layer "B.Cu") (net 12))
 (segment (start 110.72 91.24) (end 110.72 72.290991) (width 0.25) (layer "B.Cu") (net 12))
 (segment (start 108.18 68.819009) (end 107.520991 68.16) (width 0.25) (layer "B.Cu") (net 12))
 (segment (start 123.318833 99.425) (end 118.905 99.425) (width 0.25) (layer "B.Cu") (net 12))
 (segment (start 118.905 99.425) (end 110.72 91.24) (width 0.25) (layer "B.Cu") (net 12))
 (segment (start 106.589009 68.16) (end 105.64 69.109009) (width 0.25) (layer "B.Cu") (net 12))
 (segment (start 128.1 84.9) (end 126.825 86.175) (width 0.25) (layer "B.Cu") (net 12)))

